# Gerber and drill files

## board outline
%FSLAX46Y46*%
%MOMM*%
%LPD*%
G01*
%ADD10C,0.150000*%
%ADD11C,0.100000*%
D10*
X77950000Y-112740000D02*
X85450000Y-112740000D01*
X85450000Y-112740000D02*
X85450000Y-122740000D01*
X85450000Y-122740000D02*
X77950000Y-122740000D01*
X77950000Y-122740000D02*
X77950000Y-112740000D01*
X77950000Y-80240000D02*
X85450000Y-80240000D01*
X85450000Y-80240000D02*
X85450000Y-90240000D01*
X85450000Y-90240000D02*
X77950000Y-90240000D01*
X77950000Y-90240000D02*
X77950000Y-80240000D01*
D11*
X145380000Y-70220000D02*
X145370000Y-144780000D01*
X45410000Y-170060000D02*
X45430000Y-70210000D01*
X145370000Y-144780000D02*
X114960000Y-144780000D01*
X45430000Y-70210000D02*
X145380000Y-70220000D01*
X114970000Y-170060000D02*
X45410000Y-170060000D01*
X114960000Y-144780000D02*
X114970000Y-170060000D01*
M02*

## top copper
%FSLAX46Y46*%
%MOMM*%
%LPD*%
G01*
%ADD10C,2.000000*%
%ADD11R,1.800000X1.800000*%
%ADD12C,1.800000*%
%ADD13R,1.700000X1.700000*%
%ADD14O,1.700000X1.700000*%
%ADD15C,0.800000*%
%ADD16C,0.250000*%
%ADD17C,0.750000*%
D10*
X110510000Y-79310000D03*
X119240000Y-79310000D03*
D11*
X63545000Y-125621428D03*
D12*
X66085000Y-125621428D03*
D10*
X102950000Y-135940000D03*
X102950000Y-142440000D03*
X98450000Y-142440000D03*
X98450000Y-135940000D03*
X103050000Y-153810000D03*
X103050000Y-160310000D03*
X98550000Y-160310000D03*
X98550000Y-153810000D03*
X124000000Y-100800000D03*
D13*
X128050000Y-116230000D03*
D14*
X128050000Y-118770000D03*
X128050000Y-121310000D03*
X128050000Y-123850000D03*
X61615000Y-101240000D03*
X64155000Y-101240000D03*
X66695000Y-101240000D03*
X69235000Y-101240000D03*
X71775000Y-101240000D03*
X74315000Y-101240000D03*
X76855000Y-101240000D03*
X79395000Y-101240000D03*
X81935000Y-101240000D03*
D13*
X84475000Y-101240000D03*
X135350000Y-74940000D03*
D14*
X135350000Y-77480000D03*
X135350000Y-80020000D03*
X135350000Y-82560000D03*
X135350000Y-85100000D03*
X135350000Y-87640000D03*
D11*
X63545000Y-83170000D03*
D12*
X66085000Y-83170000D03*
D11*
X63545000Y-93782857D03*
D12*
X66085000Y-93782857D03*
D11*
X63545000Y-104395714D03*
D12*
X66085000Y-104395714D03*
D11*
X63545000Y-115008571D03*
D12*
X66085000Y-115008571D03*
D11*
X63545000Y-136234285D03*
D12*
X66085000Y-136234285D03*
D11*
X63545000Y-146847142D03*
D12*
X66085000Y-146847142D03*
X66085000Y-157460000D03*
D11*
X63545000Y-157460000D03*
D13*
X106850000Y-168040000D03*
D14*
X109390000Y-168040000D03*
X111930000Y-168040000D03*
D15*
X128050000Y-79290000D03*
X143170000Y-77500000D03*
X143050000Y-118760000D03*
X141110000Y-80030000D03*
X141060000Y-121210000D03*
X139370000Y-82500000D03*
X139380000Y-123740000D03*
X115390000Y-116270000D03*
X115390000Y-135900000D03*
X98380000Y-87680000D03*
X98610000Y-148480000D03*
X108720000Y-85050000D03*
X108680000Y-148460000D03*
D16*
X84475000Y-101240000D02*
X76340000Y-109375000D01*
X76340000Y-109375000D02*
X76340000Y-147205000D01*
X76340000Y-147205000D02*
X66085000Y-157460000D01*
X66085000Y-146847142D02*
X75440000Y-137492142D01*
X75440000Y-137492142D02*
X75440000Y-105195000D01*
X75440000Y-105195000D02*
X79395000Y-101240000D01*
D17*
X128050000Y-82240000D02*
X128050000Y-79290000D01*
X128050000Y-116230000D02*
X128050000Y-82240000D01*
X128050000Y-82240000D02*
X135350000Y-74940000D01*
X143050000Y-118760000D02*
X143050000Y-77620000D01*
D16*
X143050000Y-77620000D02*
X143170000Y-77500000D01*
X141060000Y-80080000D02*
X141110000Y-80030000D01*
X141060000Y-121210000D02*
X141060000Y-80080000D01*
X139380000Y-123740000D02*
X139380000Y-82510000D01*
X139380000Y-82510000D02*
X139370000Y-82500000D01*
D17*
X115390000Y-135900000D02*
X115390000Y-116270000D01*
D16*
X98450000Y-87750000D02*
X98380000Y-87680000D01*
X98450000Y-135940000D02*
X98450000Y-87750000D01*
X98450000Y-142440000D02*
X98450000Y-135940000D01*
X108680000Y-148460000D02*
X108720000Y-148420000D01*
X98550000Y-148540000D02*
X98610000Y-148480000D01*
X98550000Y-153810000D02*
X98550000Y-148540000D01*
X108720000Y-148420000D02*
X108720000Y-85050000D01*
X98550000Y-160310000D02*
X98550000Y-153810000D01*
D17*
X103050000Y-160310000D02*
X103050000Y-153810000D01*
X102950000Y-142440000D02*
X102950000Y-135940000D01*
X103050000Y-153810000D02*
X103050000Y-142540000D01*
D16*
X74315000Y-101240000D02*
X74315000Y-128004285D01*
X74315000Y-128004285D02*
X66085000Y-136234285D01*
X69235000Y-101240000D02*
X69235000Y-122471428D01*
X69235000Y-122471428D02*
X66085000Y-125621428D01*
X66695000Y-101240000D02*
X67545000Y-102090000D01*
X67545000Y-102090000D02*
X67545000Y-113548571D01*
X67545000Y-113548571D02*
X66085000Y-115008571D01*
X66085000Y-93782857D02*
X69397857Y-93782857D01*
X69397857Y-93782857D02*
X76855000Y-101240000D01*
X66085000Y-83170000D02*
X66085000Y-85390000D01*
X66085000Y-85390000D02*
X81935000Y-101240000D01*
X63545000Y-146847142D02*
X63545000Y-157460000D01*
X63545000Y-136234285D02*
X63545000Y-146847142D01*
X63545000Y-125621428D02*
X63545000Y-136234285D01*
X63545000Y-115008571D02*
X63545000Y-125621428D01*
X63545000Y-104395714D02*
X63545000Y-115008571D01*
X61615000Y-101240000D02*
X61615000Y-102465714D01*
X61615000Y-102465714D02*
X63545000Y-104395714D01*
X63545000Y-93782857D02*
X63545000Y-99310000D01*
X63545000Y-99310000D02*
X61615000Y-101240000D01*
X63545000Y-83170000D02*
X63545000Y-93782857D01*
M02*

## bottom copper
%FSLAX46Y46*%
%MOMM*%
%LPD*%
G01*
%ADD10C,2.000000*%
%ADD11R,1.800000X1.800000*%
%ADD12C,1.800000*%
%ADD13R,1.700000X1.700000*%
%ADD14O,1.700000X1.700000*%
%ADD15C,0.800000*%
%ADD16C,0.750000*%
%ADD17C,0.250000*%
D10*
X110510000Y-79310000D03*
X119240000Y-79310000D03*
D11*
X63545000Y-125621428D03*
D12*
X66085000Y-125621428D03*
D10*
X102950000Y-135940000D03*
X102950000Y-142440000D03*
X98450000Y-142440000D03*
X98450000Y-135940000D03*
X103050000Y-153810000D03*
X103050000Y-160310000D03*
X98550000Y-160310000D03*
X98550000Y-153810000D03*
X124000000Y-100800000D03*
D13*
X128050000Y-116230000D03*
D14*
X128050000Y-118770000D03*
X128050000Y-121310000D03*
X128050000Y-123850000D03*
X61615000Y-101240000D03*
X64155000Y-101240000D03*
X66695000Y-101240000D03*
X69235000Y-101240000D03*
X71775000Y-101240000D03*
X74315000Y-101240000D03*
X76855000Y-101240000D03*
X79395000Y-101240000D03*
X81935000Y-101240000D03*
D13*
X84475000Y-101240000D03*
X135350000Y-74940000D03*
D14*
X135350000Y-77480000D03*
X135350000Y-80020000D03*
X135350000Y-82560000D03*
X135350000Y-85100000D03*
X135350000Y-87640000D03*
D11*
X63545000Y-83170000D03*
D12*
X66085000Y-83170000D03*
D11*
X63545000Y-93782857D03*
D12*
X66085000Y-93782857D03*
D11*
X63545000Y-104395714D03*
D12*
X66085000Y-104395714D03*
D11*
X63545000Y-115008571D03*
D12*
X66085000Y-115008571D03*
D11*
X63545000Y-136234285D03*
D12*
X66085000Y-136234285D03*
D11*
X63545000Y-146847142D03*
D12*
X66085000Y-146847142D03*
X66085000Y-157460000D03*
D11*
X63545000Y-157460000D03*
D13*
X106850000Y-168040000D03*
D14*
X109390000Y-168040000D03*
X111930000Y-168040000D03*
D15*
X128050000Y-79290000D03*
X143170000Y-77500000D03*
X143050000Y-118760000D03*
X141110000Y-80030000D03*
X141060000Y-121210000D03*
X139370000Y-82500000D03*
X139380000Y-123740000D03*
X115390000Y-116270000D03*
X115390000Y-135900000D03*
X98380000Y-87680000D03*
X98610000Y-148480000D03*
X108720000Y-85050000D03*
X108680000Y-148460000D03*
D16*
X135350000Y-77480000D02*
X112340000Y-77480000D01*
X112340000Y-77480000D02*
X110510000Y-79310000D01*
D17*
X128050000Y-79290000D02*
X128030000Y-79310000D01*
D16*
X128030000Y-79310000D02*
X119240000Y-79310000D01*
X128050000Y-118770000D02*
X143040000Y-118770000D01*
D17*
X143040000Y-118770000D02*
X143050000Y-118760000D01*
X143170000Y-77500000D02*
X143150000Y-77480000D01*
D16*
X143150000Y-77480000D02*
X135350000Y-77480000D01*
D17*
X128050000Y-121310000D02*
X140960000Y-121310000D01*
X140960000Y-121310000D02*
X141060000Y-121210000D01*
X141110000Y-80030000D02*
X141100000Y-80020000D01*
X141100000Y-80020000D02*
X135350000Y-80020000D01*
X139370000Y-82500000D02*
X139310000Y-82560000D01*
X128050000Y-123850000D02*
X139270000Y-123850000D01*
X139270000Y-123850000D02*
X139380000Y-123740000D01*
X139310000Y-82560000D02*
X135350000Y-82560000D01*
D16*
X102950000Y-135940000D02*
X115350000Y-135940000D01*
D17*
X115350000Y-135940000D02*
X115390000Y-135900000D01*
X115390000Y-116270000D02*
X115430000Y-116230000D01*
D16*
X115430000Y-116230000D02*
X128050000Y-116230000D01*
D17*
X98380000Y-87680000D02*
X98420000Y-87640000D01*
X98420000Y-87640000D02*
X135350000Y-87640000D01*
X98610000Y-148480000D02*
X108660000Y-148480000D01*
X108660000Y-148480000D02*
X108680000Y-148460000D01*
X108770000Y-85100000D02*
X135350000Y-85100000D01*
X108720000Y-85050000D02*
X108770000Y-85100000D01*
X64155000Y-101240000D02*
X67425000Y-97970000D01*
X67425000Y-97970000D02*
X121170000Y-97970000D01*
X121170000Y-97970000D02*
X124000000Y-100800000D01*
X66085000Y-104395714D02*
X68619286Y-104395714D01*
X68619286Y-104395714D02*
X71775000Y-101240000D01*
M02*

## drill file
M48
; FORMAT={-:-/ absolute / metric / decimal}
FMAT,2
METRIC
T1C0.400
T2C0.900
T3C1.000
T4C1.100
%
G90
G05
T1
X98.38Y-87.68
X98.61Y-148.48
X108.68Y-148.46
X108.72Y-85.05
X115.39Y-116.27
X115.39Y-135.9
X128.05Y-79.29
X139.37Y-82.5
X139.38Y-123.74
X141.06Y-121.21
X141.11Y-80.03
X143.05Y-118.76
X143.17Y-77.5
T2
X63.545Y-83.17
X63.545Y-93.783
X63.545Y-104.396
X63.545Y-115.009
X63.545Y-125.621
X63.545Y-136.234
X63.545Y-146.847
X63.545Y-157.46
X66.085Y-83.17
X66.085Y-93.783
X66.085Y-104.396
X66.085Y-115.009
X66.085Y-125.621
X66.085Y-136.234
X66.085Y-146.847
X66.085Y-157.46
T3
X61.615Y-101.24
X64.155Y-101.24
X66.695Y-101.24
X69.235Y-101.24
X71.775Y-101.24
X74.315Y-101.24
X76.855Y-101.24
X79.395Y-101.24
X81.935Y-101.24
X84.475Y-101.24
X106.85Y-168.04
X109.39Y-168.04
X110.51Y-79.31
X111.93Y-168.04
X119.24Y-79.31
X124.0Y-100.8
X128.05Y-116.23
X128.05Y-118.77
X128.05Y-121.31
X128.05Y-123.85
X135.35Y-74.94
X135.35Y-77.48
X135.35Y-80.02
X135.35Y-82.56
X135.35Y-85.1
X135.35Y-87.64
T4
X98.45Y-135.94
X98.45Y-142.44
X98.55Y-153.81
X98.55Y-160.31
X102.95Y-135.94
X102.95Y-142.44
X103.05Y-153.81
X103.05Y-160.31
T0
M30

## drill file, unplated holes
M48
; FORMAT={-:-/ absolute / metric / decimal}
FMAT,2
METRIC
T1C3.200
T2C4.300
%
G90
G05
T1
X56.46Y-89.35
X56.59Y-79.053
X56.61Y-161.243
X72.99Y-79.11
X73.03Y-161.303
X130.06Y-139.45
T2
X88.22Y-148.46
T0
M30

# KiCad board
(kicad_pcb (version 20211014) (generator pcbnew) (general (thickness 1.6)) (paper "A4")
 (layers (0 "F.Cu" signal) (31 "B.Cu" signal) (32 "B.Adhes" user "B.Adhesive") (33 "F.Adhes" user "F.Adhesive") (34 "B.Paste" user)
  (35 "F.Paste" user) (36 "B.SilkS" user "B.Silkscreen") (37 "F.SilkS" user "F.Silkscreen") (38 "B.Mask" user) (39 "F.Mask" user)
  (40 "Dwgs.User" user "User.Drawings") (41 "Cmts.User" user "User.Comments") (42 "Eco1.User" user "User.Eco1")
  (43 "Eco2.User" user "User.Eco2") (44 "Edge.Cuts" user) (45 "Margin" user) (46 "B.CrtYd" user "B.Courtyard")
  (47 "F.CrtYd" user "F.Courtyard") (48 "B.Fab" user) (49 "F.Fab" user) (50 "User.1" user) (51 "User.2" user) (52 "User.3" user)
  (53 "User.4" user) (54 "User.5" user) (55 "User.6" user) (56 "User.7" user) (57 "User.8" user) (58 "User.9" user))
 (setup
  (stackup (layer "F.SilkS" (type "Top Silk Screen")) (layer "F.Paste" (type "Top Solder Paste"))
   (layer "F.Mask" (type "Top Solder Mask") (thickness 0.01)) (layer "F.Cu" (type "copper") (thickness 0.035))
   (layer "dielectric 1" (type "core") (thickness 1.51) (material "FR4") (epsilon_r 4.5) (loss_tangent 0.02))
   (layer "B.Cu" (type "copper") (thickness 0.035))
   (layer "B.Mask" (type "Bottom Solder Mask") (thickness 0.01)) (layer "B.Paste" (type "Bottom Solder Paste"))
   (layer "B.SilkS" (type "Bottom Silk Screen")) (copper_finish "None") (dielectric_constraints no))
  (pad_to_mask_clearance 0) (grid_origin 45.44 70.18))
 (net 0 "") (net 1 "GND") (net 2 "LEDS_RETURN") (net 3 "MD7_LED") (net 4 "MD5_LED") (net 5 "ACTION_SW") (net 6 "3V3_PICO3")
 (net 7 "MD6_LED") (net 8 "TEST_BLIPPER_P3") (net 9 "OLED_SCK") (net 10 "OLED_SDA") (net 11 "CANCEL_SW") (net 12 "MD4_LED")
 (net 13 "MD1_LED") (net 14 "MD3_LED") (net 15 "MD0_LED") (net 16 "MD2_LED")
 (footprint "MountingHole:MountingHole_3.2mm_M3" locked (layer "F.Cu") (at 130.06 139.450113)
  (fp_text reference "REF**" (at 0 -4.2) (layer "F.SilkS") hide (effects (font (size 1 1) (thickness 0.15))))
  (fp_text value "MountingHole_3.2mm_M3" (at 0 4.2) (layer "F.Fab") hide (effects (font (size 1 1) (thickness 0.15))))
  (pad "" np_thru_hole circle locked (at 0 0) (size 3.2 3.2) (drill 3.2) (layers *.Cu *.Mask)))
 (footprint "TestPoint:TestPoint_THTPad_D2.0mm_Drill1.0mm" (layer "F.Cu") (at 119.24 79.31)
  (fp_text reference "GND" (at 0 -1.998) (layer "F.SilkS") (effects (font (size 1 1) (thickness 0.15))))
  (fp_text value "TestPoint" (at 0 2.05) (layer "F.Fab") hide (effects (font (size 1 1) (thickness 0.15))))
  (pad "1" thru_hole circle (at 0 0) (size 2 2) (drill 1) (layers *.Cu *.Mask) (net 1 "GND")))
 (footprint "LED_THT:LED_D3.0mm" (layer "F.Cu") (at 63.545 115.008571)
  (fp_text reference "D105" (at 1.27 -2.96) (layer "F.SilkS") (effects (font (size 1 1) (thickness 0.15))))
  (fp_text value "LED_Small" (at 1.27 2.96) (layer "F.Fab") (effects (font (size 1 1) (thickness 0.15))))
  (pad "1" thru_hole rect (at 0 0) (size 1.8 1.8) (drill 0.9) (layers *.Cu *.Mask) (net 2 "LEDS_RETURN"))
  (pad "2" thru_hole circle (at 2.54 0) (size 1.8 1.8) (drill 0.9) (layers *.Cu *.Mask) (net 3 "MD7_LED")))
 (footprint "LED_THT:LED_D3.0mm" (layer "F.Cu") (at 63.545 104.395714)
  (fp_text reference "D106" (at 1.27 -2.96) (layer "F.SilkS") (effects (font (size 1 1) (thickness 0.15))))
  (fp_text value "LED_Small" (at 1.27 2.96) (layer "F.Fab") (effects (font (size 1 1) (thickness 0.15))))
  (pad "1" thru_hole rect (at 0 0) (size 1.8 1.8) (drill 0.9) (layers *.Cu *.Mask) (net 2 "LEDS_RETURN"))
  (pad "2" thru_hole circle (at 2.54 0) (size 1.8 1.8) (drill 0.9) (layers *.Cu *.Mask) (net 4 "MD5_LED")))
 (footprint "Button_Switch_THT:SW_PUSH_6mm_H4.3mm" (layer "F.Cu") (at 98.55 160.31 90)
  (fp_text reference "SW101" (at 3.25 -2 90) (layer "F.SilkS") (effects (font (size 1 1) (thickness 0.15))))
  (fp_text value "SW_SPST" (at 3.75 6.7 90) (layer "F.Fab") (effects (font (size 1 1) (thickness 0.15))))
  (pad "1" thru_hole circle (at 0 0 180) (size 2 2) (drill 1.1) (layers *.Cu *.Mask) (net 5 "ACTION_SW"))
  (pad "1" thru_hole circle (at 6.5 0 180) (size 2 2) (drill 1.1) (layers *.Cu *.Mask) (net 5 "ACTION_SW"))
  (pad "2" thru_hole circle (at 0 4.5 180) (size 2 2) (drill 1.1) (layers *.Cu *.Mask) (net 1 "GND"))
  (pad "2" thru_hole circle (at 6.5 4.5 180) (size 2 2) (drill 1.1) (layers *.Cu *.Mask) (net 1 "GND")))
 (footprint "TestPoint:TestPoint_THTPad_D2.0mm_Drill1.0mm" (layer "F.Cu") (at 110.51 79.31)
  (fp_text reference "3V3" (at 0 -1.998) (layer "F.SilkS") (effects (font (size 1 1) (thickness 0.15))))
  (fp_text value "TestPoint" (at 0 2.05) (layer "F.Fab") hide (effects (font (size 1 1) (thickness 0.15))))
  (pad "1" thru_hole circle (at 0 0) (size 2 2) (drill 1) (layers *.Cu *.Mask) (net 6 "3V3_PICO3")))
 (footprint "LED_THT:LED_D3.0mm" (layer "F.Cu") (at 63.545 125.621428)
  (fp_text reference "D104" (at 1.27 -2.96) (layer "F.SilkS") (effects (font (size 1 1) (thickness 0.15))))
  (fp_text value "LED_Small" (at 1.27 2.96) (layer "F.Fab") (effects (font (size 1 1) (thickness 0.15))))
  (pad "1" thru_hole rect (at 0 0) (size 1.8 1.8) (drill 0.9) (layers *.Cu *.Mask) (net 2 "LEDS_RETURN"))
  (pad "2" thru_hole circle (at 2.54 0) (size 1.8 1.8) (drill 0.9) (layers *.Cu *.Mask) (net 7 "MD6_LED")))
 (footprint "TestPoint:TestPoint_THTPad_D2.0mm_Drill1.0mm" (layer "F.Cu") (at 124 100.8)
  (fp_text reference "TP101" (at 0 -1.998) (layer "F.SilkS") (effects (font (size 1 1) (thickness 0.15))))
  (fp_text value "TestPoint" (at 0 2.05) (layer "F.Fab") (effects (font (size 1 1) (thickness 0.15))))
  (pad "1" thru_hole circle (at 0 0) (size 2 2) (drill 1) (layers *.Cu *.Mask) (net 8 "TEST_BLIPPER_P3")))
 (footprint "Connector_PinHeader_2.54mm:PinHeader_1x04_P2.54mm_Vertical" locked (layer "F.Cu") (at 128.05 116.23)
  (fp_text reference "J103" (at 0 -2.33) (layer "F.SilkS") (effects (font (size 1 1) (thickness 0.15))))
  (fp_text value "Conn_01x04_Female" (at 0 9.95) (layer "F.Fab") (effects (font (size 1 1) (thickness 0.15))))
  (pad "1" thru_hole rect locked (at 0 0) (size 1.7 1.7) (drill 1) (layers *.Cu *.Mask) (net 1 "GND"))
  (pad "2" thru_hole oval locked (at 0 2.54) (size 1.7 1.7) (drill 1) (layers *.Cu *.Mask) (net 6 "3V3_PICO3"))
  (pad "3" thru_hole oval locked (at 0 5.08) (size 1.7 1.7) (drill 1) (layers *.Cu *.Mask) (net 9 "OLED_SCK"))
  (pad "4" thru_hole oval locked (at 0 7.62) (size 1.7 1.7) (drill 1) (layers *.Cu *.Mask) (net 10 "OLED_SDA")))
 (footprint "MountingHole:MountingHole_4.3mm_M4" (layer "F.Cu") (at 88.22 148.46)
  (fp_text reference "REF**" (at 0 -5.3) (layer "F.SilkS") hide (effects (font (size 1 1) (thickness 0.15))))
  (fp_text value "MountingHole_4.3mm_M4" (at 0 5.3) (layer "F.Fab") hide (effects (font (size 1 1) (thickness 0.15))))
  (pad "" np_thru_hole circle (at 0 0) (size 4.3 4.3) (drill 4.3) (layers F&B.Cu *.Mask)))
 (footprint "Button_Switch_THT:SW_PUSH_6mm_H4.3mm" (layer "F.Cu") (at 98.45 142.44 90)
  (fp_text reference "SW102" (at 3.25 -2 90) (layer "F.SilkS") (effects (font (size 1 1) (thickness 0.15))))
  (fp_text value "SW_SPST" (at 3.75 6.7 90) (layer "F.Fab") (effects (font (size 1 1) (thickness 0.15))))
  (pad "1" thru_hole circle (at 6.5 0 180) (size 2 2) (drill 1.1) (layers *.Cu *.Mask) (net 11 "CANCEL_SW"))
  (pad "1" thru_hole circle (at 0 0 180) (size 2 2) (drill 1.1) (layers *.Cu *.Mask) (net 11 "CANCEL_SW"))
  (pad "2" thru_hole circle (at 6.5 4.5 180) (size 2 2) (drill 1.1) (layers *.Cu *.Mask) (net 1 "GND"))
  (pad "2" thru_hole circle (at 0 4.5 180) (size 2 2) (drill 1.1) (layers *.Cu *.Mask) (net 1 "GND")))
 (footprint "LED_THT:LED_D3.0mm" (layer "F.Cu") (at 63.545 136.234285)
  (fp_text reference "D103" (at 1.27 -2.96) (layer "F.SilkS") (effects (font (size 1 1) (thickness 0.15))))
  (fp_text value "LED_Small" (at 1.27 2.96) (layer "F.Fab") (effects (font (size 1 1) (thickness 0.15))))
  (pad "1" thru_hole rect (at 0 0) (size 1.8 1.8) (drill 0.9) (layers *.Cu *.Mask) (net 2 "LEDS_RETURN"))
  (pad "2" thru_hole circle (at 2.54 0) (size 1.8 1.8) (drill 0.9) (layers *.Cu *.Mask) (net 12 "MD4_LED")))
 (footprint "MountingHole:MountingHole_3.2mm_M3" (layer "F.Cu") (at 56.59 79.052856 -90)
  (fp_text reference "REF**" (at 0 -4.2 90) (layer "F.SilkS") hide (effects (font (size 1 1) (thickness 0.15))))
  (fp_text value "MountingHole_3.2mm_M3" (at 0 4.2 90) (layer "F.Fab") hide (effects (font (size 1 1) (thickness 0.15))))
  (pad "" np_thru_hole circle locked (at 0 0 270) (size 3.2 3.2) (drill 3.2) (layers F&B.Cu *.Mask)))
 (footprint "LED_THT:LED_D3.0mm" (layer "F.Cu") (at 63.545 83.17)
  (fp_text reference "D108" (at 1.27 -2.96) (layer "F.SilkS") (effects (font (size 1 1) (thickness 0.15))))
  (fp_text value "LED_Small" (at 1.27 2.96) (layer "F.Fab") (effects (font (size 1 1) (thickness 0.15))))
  (pad "1" thru_hole rect (at 0 0) (size 1.8 1.8) (drill 0.9) (layers *.Cu *.Mask) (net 2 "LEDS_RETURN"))
  (pad "2" thru_hole circle (at 2.54 0) (size 1.8 1.8) (drill 0.9) (layers *.Cu *.Mask) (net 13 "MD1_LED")))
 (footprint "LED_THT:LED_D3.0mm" (layer "F.Cu") (at 63.545 93.782857)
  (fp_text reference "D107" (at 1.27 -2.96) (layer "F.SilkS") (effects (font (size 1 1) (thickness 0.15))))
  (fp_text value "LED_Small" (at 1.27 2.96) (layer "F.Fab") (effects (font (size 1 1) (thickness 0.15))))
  (pad "1" thru_hole rect (at 0 0) (size 1.8 1.8) (drill 0.9) (layers *.Cu *.Mask) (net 2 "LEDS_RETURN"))
  (pad "2" thru_hole circle (at 2.54 0) (size 1.8 1.8) (drill 0.9) (layers *.Cu *.Mask) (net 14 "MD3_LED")))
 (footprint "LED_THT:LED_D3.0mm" (layer "F.Cu") (at 63.545 157.46)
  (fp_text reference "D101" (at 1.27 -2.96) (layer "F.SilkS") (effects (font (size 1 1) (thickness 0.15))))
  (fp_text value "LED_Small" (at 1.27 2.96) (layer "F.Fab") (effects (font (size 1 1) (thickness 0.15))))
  (pad "1" thru_hole rect (at 0 0) (size 1.8 1.8) (drill 0.9) (layers *.Cu *.Mask) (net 2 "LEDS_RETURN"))
  (pad "2" thru_hole circle (at 2.54 0) (size 1.8 1.8) (drill 0.9) (layers *.Cu *.Mask) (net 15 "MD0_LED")))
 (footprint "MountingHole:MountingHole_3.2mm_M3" (layer "F.Cu") (at 56.61 161.242856 -90)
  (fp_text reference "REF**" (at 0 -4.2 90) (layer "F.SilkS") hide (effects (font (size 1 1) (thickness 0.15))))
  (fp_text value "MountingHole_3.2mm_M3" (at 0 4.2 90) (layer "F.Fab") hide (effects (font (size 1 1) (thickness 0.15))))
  (pad "" np_thru_hole circle locked (at 0 0 270) (size 3.2 3.2) (drill 3.2) (layers F&B.Cu *.Mask)))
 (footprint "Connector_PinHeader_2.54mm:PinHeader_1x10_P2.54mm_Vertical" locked (layer "F.Cu") (at 84.475 101.24 -90)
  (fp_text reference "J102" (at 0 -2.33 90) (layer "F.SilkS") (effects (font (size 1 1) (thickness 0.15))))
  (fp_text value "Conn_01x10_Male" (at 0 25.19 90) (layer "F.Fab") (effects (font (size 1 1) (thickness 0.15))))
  (pad "1" thru_hole rect locked (at 0 0 270) (size 1.7 1.7) (drill 1) (layers *.Cu *.Mask) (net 15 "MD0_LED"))
  (pad "2" thru_hole oval locked (at 0 2.54 270) (size 1.7 1.7) (drill 1) (layers *.Cu *.Mask) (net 13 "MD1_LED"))
  (pad "3" thru_hole oval locked (at 0 5.08 270) (size 1.7 1.7) (drill 1) (layers *.Cu *.Mask) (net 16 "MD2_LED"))
  (pad "4" thru_hole oval locked (at 0 7.62 270) (size 1.7 1.7) (drill 1) (layers *.Cu *.Mask) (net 14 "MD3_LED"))
  (pad "5" thru_hole oval locked (at 0 10.16 270) (size 1.7 1.7) (drill 1) (layers *.Cu *.Mask) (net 12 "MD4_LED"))
  (pad "6" thru_hole oval locked (at 0 12.7 270) (size 1.7 1.7) (drill 1) (layers *.Cu *.Mask) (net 4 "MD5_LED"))
  (pad "7" thru_hole oval locked (at 0 15.24 270) (size 1.7 1.7) (drill 1) (layers *.Cu *.Mask) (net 7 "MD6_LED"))
  (pad "8" thru_hole oval locked (at 0 17.78 270) (size 1.7 1.7) (drill 1) (layers *.Cu *.Mask) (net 3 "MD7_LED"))
  (pad "9" thru_hole oval locked (at 0 20.32 270) (size 1.7 1.7) (drill 1) (layers *.Cu *.Mask) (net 8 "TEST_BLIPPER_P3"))
  (pad "10" thru_hole oval locked (at 0 22.86 270) (size 1.7 1.7) (drill 1) (layers *.Cu *.Mask) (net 2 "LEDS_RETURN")))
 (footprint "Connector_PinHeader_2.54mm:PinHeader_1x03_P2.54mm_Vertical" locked (layer "F.Cu") (at 106.85 168.04 90)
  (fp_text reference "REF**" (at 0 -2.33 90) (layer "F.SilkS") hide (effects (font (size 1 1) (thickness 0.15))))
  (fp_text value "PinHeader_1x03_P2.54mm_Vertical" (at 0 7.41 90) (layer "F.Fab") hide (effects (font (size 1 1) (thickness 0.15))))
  (pad "1" thru_hole rect locked (at 0 0 90) (size 1.7 1.7) (drill 1) (layers F&B.Cu *.Mask))
  (pad "2" thru_hole oval locked (at 0 2.54 90) (size 1.7 1.7) (drill 1) (layers F&B.Cu *.Mask))
  (pad "3" thru_hole oval locked (at 0 5.08 90) (size 1.7 1.7) (drill 1) (layers F&B.Cu *.Mask)))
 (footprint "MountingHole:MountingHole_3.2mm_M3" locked (layer "F.Cu") (at 56.46 89.350113)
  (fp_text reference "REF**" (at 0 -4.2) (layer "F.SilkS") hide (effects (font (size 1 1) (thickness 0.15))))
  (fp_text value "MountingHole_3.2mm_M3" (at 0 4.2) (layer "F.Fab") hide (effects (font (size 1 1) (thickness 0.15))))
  (pad "" np_thru_hole circle locked (at 0 0) (size 3.2 3.2) (drill 3.2) (layers *.Cu *.Mask)))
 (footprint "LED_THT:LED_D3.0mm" (layer "F.Cu") (at 63.545 146.847142)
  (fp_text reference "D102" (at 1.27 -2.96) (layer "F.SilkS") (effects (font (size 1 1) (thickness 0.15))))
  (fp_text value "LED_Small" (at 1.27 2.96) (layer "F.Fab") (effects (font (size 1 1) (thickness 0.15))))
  (pad "1" thru_hole rect (at 0 0) (size 1.8 1.8) (drill 0.9) (layers *.Cu *.Mask) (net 2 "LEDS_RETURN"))
  (pad "2" thru_hole circle (at 2.54 0) (size 1.8 1.8) (drill 0.9) (layers *.Cu *.Mask) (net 16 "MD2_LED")))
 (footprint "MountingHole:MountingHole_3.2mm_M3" (layer "F.Cu") (at 73.03 161.302856 -90)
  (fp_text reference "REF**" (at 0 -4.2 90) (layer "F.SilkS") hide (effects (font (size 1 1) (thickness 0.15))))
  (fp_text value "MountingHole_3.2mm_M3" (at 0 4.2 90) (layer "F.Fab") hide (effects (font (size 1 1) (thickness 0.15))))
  (pad "" np_thru_hole circle locked (at 0 0 270) (size 3.2 3.2) (drill 3.2) (layers F&B.Cu *.Mask)))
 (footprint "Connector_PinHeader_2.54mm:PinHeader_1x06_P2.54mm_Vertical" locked (layer "F.Cu") (at 135.35 74.94)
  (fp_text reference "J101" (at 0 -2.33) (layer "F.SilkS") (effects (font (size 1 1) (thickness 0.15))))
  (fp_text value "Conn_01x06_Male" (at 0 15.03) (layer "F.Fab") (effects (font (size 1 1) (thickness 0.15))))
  (pad "1" thru_hole rect locked (at 0 0) (size 1.7 1.7) (drill 1) (layers *.Cu *.Mask) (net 1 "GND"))
  (pad "2" thru_hole oval locked (at 0 2.54) (size 1.7 1.7) (drill 1) (layers *.Cu *.Mask) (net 6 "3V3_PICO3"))
  (pad "3" thru_hole oval locked (at 0 5.08) (size 1.7 1.7) (drill 1) (layers *.Cu *.Mask) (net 9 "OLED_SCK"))
  (pad "4" thru_hole oval locked (at 0 7.62) (size 1.7 1.7) (drill 1) (layers *.Cu *.Mask) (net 10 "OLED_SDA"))
  (pad "5" thru_hole oval locked (at 0 10.16) (size 1.7 1.7) (drill 1) (layers *.Cu *.Mask) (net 5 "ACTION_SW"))
  (pad "6" thru_hole oval locked (at 0 12.7) (size 1.7 1.7) (drill 1) (layers *.Cu *.Mask) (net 11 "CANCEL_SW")))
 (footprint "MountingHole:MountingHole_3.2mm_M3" (layer "F.Cu") (at 72.99 79.11)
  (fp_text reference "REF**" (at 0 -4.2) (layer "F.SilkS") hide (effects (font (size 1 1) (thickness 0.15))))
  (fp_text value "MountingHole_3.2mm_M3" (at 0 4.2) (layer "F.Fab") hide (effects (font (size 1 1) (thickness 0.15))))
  (pad "" np_thru_hole circle locked (at 0 0) (size 3.2 3.2) (drill 3.2) (layers F&B.Cu *.Mask)))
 (gr_line (start 145.37 144.78) (end 114.96 144.78) (layer "Edge.Cuts") (width 0.1))
 (gr_line (start 114.97 170.06) (end 45.41 170.06) (layer "Edge.Cuts") (width 0.1))
 (gr_rect (start 77.95 80.24) (end 85.45 90.24) (layer "Edge.Cuts") (width 0.15) (fill none))
 (gr_line (start 145.38 70.22) (end 145.37 144.78) (layer "Edge.Cuts") (width 0.1))
 (gr_line (start 114.96 144.78) (end 114.97 170.06) (layer "Edge.Cuts") (width 0.1))
 (gr_rect (start 77.95 112.74) (end 85.45 122.74) (layer "Edge.Cuts") (width 0.15) (fill none))
 (gr_line (start 45.43 70.21) (end 145.38 70.22) (layer "Edge.Cuts") (width 0.1))
 (gr_line (start 45.41 170.06) (end 45.43 70.21) (layer "Edge.Cuts") (width 0.1))
 (segment (start 63.545 104.395714) (end 63.545 115.008571) (width 0.25) (layer "F.Cu") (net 2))
 (segment (start 61.615 102.465714) (end 63.545 104.395714) (width 0.25) (layer "F.Cu") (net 2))
 (segment (start 63.545 125.621428) (end 63.545 136.234285) (width 0.25) (layer "F.Cu") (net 2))
 (segment (start 63.545 83.17) (end 63.545 93.782857) (width 0.25) (layer "F.Cu") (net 2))
 (segment (start 63.545 146.847142) (end 63.545 157.46) (width 0.25) (layer "F.Cu") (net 2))
 (segment (start 63.545 93.782857) (end 63.545 99.31) (width 0.25) (layer "F.Cu") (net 2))
 (segment (start 61.615 101.24) (end 61.615 102.465714) (width 0.25) (layer "F.Cu") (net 2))
 (segment (start 63.545 136.234285) (end 63.545 146.847142) (width 0.25) (layer "F.Cu") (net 2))
 (segment (start 63.545 99.31) (end 61.615 101.24) (width 0.25) (layer "F.Cu") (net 2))
 (segment (start 63.545 115.008571) (end 63.545 125.621428) (width 0.25) (layer "F.Cu") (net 2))
 (segment (start 76.34 109.375) (end 76.34 147.205) (width 0.25) (layer "F.Cu") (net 15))
 (segment (start 84.475 101.24) (end 76.34 109.375) (width 0.25) (layer "F.Cu") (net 15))
 (segment (start 76.34 147.205) (end 66.085 157.46) (width 0.25) (layer "F.Cu") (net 15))
 (segment (start 75.44 105.195) (end 79.395 101.24) (width 0.25) (layer "F.Cu") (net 16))
 (segment (start 75.44 137.492142) (end 75.44 105.195) (width 0.25) (layer "F.Cu") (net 16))
 (segment (start 66.085 146.847142) (end 75.44 137.492142) (width 0.25) (layer "F.Cu") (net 16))
 (segment (start 74.315 128.004285) (end 66.085 136.234285) (width 0.25) (layer "F.Cu") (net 12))
 (segment (start 74.315 101.24) (end 74.315 128.004285) (width 0.25) (layer "F.Cu") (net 12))
 (segment (start 69.235 101.24) (end 69.235 122.471428) (width 0.25) (layer "F.Cu") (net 7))
 (segment (start 69.235 122.471428) (end 66.085 125.621428) (width 0.25) (layer "F.Cu") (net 7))
 (segment (start 67.545 113.548571) (end 66.085 115.008571) (width 0.25) (layer "F.Cu") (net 3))
 (segment (start 67.545 102.09) (end 67.545 113.548571) (width 0.25) (layer "F.Cu") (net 3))
 (segment (start 66.695 101.24) (end 67.545 102.09) (width 0.25) (layer "F.Cu") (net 3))
 (segment (start 66.085 104.395714) (end 68.619286 104.395714) (width 0.25) (layer "B.Cu") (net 4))
 (segment (start 68.619286 104.395714) (end 71.775 101.24) (width 0.25) (layer "B.Cu") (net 4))
 (segment (start 66.085 93.782857) (end 69.397857 93.782857) (width 0.25) (layer "F.Cu") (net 14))
 (segment (start 69.397857 93.782857) (end 76.855 101.24) (width 0.25) (layer "F.Cu") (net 14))
 (segment (start 66.085 85.39) (end 81.935 101.24) (width 0.25) (layer "F.Cu") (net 13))
 (segment (start 66.085 83.17) (end 66.085 85.39) (width 0.25) (layer "F.Cu") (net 13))
 (segment (start 115.39 135.9) (end 115.39 116.27) (width 0.75) (layer "F.Cu") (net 1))
 (segment (start 103.05 153.81) (end 103.05 142.54) (width 0.75) (layer "F.Cu") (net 1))
 (segment (start 103.05 160.31) (end 103.05 153.81) (width 0.75) (layer "F.Cu") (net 1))
 (segment (start 128.05 116.23) (end 128.05 82.24) (width 0.75) (layer "F.Cu") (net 1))
 (segment (start 128.05 82.24) (end 135.35 74.94) (width 0.75) (layer "F.Cu") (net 1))
 (segment (start 128.05 82.24) (end 128.05 79.29) (width 0.75) (layer "F.Cu") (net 1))
 (segment (start 102.95 142.44) (end 102.95 135.94) (width 0.75) (layer "F.Cu") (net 1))
 (via (at 115.39 135.9) (size 0.8) (drill 0.4) (layers "F.Cu" "B.Cu") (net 1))
 (via (at 128.05 79.29) (size 0.8) (drill 0.4) (layers "F.Cu" "B.Cu") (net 1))
 (via (at 115.39 116.27) (size 0.8) (drill 0.4) (layers "F.Cu" "B.Cu") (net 1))
 (segment (start 102.95 135.94) (end 115.35 135.94) (width 0.75) (layer "B.Cu") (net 1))
 (segment (start 115.43 116.23) (end 128.05 116.23) (width 0.75) (layer "B.Cu") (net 1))
 (segment (start 128.05 79.29) (end 128.03 79.31) (width 0.25) (layer "B.Cu") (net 1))
 (segment (start 128.03 79.31) (end 119.24 79.31) (width 0.75) (layer "B.Cu") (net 1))
 (segment (start 115.35 135.94) (end 115.39 135.9) (width 0.25) (layer "B.Cu") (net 1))
 (segment (start 115.39 116.27) (end 115.43 116.23) (width 0.25) (layer "B.Cu") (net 1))
 (segment (start 143.05 118.76) (end 143.05 77.62) (width 0.75) (layer "F.Cu") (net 6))
 (segment (start 143.05 77.62) (end 143.17 77.5) (width 0.25) (layer "F.Cu") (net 6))
 (via (at 143.17 77.5) (size 0.8) (drill 0.4) (layers "F.Cu" "B.Cu") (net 6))
 (via (at 143.05 118.76) (size 0.8) (drill 0.4) (layers "F.Cu" "B.Cu") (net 6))
 (segment (start 135.35 77.48) (end 112.34 77.48) (width 0.75) (layer "B.Cu") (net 6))
 (segment (start 143.17 77.5) (end 143.15 77.48) (width 0.25) (layer "B.Cu") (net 6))
 (segment (start 128.05 118.77) (end 143.04 118.77) (width 0.75) (layer "B.Cu") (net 6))
 (segment (start 143.04 118.77) (end 143.05 118.76) (width 0.25) (layer "B.Cu") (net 6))
 (segment (start 112.34 77.48) (end 110.51 79.31) (width 0.75) (layer "B.Cu") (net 6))
 (segment (start 143.15 77.48) (end 135.35 77.48) (width 0.75) (layer "B.Cu") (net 6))
 (segment (start 141.06 80.08) (end 141.11 80.03) (width 0.25) (layer "F.Cu") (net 9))
 (segment (start 141.06 121.21) (end 141.06 80.08) (width 0.25) (layer "F.Cu") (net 9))
 (via (at 141.11 80.03) (size 0.8) (drill 0.4) (layers "F.Cu" "B.Cu") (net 9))
 (via (at 141.06 121.21) (size 0.8) (drill 0.4) (layers "F.Cu" "B.Cu") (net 9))
 (segment (start 141.11 80.03) (end 141.1 80.02) (width 0.25) (layer "B.Cu") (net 9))
 (segment (start 140.96 121.31) (end 141.06 121.21) (width 0.25) (layer "B.Cu") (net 9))
 (segment (start 141.1 80.02) (end 135.35 80.02) (width 0.25) (layer "B.Cu") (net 9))
 (segment (start 128.05 121.31) (end 140.96 121.31) (width 0.25) (layer "B.Cu") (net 9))
 (segment (start 139.38 123.74) (end 139.38 82.51) (width 0.25) (layer "F.Cu") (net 10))
 (segment (start 139.38 82.51) (end 139.37 82.5) (width 0.25) (layer "F.Cu") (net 10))
 (via (at 139.37 82.5) (size 0.8) (drill 0.4) (layers "F.Cu" "B.Cu") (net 10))
 (via (at 139.38 123.74) (size 0.8) (drill 0.4) (layers "F.Cu" "B.Cu") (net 10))
 (segment (start 139.37 82.5) (end 139.31 82.56) (width 0.25) (layer "B.Cu") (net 10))
 (segment (start 139.31 82.56) (end 135.35 82.56) (width 0.25) (layer "B.Cu") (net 10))
 (segment (start 139.27 123.85) (end 139.38 123.74) (width 0.25) (layer "B.Cu") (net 10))
 (segment (start 128.05 123.85) (end 139.27 123.85) (width 0.25) (layer "B.Cu") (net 10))
 (segment (start 98.55 153.81) (end 98.55 148.54) (width 0.25) (layer "F.Cu") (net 5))
 (segment (start 98.55 160.31) (end 98.55 153.81) (width 0.25) (layer "F.Cu") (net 5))
 (segment (start 108.68 148.46) (end 108.72 148.42) (width 0.25) (layer "F.Cu") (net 5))
 (segment (start 98.55 148.54) (end 98.61 148.48) (width 0.25) (layer "F.Cu") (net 5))
 (segment (start 108.72 148.42) (end 108.72 85.05) (width 0.25) (layer "F.Cu") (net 5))
 (via (at 108.72 85.05) (size 0.8) (drill 0.4) (layers "F.Cu" "B.Cu") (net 5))
 (via (at 108.68 148.46) (size 0.8) (drill 0.4) (layers "F.Cu" "B.Cu") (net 5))
 (via (at 98.61 148.48) (size 0.8) (drill 0.4) (layers "F.Cu" "B.Cu") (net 5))
 (segment (start 108.66 148.48) (end 108.68 148.46) (width 0.25) (layer "B.Cu") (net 5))
 (segment (start 108.72 85.05) (end 108.77 85.1) (width 0.25) (layer "B.Cu") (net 5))
 (segment (start 98.61 148.48) (end 108.66 148.48) (width 0.25) (layer "B.Cu") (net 5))
 (segment (start 108.77 85.1) (end 135.35 85.1) (width 0.25) (layer "B.Cu") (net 5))
 (segment (start 98.45 135.94) (end 98.45 87.75) (width 0.25) (layer "F.Cu") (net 11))
 (segment (start 98.45 87.75) (end 98.38 87.68) (width 0.25) (layer "F.Cu") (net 11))
 (segment (start 98.45 142.44) (end 98.45 135.94) (width 0.25) (layer "F.Cu") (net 11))
 (via (at 98.38 87.68) (size 0.8) (drill 0.4) (layers "F.Cu" "B.Cu") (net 11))
 (segment (start 98.38 87.68) (end 98.42 87.64) (width 0.25) (layer "B.Cu") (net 11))
 (segment (start 98.42 87.64) (end 135.35 87.64) (width 0.25) (layer "B.Cu") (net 11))
 (segment (start 64.155 101.24) (end 67.425 97.97) (width 0.25) (layer "B.Cu") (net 8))
 (segment (start 67.425 97.97) (end 121.17 97.97) (width 0.25) (layer "B.Cu") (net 8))
 (segment (start 121.17 97.97) (end 124 100.8) (width 0.25) (layer "B.Cu") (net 8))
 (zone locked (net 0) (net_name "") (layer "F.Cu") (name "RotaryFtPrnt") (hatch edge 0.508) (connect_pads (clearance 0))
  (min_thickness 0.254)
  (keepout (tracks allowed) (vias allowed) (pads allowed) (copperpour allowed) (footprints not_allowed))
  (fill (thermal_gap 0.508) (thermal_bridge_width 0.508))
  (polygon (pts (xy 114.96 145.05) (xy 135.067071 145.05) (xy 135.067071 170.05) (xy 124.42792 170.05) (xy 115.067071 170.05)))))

